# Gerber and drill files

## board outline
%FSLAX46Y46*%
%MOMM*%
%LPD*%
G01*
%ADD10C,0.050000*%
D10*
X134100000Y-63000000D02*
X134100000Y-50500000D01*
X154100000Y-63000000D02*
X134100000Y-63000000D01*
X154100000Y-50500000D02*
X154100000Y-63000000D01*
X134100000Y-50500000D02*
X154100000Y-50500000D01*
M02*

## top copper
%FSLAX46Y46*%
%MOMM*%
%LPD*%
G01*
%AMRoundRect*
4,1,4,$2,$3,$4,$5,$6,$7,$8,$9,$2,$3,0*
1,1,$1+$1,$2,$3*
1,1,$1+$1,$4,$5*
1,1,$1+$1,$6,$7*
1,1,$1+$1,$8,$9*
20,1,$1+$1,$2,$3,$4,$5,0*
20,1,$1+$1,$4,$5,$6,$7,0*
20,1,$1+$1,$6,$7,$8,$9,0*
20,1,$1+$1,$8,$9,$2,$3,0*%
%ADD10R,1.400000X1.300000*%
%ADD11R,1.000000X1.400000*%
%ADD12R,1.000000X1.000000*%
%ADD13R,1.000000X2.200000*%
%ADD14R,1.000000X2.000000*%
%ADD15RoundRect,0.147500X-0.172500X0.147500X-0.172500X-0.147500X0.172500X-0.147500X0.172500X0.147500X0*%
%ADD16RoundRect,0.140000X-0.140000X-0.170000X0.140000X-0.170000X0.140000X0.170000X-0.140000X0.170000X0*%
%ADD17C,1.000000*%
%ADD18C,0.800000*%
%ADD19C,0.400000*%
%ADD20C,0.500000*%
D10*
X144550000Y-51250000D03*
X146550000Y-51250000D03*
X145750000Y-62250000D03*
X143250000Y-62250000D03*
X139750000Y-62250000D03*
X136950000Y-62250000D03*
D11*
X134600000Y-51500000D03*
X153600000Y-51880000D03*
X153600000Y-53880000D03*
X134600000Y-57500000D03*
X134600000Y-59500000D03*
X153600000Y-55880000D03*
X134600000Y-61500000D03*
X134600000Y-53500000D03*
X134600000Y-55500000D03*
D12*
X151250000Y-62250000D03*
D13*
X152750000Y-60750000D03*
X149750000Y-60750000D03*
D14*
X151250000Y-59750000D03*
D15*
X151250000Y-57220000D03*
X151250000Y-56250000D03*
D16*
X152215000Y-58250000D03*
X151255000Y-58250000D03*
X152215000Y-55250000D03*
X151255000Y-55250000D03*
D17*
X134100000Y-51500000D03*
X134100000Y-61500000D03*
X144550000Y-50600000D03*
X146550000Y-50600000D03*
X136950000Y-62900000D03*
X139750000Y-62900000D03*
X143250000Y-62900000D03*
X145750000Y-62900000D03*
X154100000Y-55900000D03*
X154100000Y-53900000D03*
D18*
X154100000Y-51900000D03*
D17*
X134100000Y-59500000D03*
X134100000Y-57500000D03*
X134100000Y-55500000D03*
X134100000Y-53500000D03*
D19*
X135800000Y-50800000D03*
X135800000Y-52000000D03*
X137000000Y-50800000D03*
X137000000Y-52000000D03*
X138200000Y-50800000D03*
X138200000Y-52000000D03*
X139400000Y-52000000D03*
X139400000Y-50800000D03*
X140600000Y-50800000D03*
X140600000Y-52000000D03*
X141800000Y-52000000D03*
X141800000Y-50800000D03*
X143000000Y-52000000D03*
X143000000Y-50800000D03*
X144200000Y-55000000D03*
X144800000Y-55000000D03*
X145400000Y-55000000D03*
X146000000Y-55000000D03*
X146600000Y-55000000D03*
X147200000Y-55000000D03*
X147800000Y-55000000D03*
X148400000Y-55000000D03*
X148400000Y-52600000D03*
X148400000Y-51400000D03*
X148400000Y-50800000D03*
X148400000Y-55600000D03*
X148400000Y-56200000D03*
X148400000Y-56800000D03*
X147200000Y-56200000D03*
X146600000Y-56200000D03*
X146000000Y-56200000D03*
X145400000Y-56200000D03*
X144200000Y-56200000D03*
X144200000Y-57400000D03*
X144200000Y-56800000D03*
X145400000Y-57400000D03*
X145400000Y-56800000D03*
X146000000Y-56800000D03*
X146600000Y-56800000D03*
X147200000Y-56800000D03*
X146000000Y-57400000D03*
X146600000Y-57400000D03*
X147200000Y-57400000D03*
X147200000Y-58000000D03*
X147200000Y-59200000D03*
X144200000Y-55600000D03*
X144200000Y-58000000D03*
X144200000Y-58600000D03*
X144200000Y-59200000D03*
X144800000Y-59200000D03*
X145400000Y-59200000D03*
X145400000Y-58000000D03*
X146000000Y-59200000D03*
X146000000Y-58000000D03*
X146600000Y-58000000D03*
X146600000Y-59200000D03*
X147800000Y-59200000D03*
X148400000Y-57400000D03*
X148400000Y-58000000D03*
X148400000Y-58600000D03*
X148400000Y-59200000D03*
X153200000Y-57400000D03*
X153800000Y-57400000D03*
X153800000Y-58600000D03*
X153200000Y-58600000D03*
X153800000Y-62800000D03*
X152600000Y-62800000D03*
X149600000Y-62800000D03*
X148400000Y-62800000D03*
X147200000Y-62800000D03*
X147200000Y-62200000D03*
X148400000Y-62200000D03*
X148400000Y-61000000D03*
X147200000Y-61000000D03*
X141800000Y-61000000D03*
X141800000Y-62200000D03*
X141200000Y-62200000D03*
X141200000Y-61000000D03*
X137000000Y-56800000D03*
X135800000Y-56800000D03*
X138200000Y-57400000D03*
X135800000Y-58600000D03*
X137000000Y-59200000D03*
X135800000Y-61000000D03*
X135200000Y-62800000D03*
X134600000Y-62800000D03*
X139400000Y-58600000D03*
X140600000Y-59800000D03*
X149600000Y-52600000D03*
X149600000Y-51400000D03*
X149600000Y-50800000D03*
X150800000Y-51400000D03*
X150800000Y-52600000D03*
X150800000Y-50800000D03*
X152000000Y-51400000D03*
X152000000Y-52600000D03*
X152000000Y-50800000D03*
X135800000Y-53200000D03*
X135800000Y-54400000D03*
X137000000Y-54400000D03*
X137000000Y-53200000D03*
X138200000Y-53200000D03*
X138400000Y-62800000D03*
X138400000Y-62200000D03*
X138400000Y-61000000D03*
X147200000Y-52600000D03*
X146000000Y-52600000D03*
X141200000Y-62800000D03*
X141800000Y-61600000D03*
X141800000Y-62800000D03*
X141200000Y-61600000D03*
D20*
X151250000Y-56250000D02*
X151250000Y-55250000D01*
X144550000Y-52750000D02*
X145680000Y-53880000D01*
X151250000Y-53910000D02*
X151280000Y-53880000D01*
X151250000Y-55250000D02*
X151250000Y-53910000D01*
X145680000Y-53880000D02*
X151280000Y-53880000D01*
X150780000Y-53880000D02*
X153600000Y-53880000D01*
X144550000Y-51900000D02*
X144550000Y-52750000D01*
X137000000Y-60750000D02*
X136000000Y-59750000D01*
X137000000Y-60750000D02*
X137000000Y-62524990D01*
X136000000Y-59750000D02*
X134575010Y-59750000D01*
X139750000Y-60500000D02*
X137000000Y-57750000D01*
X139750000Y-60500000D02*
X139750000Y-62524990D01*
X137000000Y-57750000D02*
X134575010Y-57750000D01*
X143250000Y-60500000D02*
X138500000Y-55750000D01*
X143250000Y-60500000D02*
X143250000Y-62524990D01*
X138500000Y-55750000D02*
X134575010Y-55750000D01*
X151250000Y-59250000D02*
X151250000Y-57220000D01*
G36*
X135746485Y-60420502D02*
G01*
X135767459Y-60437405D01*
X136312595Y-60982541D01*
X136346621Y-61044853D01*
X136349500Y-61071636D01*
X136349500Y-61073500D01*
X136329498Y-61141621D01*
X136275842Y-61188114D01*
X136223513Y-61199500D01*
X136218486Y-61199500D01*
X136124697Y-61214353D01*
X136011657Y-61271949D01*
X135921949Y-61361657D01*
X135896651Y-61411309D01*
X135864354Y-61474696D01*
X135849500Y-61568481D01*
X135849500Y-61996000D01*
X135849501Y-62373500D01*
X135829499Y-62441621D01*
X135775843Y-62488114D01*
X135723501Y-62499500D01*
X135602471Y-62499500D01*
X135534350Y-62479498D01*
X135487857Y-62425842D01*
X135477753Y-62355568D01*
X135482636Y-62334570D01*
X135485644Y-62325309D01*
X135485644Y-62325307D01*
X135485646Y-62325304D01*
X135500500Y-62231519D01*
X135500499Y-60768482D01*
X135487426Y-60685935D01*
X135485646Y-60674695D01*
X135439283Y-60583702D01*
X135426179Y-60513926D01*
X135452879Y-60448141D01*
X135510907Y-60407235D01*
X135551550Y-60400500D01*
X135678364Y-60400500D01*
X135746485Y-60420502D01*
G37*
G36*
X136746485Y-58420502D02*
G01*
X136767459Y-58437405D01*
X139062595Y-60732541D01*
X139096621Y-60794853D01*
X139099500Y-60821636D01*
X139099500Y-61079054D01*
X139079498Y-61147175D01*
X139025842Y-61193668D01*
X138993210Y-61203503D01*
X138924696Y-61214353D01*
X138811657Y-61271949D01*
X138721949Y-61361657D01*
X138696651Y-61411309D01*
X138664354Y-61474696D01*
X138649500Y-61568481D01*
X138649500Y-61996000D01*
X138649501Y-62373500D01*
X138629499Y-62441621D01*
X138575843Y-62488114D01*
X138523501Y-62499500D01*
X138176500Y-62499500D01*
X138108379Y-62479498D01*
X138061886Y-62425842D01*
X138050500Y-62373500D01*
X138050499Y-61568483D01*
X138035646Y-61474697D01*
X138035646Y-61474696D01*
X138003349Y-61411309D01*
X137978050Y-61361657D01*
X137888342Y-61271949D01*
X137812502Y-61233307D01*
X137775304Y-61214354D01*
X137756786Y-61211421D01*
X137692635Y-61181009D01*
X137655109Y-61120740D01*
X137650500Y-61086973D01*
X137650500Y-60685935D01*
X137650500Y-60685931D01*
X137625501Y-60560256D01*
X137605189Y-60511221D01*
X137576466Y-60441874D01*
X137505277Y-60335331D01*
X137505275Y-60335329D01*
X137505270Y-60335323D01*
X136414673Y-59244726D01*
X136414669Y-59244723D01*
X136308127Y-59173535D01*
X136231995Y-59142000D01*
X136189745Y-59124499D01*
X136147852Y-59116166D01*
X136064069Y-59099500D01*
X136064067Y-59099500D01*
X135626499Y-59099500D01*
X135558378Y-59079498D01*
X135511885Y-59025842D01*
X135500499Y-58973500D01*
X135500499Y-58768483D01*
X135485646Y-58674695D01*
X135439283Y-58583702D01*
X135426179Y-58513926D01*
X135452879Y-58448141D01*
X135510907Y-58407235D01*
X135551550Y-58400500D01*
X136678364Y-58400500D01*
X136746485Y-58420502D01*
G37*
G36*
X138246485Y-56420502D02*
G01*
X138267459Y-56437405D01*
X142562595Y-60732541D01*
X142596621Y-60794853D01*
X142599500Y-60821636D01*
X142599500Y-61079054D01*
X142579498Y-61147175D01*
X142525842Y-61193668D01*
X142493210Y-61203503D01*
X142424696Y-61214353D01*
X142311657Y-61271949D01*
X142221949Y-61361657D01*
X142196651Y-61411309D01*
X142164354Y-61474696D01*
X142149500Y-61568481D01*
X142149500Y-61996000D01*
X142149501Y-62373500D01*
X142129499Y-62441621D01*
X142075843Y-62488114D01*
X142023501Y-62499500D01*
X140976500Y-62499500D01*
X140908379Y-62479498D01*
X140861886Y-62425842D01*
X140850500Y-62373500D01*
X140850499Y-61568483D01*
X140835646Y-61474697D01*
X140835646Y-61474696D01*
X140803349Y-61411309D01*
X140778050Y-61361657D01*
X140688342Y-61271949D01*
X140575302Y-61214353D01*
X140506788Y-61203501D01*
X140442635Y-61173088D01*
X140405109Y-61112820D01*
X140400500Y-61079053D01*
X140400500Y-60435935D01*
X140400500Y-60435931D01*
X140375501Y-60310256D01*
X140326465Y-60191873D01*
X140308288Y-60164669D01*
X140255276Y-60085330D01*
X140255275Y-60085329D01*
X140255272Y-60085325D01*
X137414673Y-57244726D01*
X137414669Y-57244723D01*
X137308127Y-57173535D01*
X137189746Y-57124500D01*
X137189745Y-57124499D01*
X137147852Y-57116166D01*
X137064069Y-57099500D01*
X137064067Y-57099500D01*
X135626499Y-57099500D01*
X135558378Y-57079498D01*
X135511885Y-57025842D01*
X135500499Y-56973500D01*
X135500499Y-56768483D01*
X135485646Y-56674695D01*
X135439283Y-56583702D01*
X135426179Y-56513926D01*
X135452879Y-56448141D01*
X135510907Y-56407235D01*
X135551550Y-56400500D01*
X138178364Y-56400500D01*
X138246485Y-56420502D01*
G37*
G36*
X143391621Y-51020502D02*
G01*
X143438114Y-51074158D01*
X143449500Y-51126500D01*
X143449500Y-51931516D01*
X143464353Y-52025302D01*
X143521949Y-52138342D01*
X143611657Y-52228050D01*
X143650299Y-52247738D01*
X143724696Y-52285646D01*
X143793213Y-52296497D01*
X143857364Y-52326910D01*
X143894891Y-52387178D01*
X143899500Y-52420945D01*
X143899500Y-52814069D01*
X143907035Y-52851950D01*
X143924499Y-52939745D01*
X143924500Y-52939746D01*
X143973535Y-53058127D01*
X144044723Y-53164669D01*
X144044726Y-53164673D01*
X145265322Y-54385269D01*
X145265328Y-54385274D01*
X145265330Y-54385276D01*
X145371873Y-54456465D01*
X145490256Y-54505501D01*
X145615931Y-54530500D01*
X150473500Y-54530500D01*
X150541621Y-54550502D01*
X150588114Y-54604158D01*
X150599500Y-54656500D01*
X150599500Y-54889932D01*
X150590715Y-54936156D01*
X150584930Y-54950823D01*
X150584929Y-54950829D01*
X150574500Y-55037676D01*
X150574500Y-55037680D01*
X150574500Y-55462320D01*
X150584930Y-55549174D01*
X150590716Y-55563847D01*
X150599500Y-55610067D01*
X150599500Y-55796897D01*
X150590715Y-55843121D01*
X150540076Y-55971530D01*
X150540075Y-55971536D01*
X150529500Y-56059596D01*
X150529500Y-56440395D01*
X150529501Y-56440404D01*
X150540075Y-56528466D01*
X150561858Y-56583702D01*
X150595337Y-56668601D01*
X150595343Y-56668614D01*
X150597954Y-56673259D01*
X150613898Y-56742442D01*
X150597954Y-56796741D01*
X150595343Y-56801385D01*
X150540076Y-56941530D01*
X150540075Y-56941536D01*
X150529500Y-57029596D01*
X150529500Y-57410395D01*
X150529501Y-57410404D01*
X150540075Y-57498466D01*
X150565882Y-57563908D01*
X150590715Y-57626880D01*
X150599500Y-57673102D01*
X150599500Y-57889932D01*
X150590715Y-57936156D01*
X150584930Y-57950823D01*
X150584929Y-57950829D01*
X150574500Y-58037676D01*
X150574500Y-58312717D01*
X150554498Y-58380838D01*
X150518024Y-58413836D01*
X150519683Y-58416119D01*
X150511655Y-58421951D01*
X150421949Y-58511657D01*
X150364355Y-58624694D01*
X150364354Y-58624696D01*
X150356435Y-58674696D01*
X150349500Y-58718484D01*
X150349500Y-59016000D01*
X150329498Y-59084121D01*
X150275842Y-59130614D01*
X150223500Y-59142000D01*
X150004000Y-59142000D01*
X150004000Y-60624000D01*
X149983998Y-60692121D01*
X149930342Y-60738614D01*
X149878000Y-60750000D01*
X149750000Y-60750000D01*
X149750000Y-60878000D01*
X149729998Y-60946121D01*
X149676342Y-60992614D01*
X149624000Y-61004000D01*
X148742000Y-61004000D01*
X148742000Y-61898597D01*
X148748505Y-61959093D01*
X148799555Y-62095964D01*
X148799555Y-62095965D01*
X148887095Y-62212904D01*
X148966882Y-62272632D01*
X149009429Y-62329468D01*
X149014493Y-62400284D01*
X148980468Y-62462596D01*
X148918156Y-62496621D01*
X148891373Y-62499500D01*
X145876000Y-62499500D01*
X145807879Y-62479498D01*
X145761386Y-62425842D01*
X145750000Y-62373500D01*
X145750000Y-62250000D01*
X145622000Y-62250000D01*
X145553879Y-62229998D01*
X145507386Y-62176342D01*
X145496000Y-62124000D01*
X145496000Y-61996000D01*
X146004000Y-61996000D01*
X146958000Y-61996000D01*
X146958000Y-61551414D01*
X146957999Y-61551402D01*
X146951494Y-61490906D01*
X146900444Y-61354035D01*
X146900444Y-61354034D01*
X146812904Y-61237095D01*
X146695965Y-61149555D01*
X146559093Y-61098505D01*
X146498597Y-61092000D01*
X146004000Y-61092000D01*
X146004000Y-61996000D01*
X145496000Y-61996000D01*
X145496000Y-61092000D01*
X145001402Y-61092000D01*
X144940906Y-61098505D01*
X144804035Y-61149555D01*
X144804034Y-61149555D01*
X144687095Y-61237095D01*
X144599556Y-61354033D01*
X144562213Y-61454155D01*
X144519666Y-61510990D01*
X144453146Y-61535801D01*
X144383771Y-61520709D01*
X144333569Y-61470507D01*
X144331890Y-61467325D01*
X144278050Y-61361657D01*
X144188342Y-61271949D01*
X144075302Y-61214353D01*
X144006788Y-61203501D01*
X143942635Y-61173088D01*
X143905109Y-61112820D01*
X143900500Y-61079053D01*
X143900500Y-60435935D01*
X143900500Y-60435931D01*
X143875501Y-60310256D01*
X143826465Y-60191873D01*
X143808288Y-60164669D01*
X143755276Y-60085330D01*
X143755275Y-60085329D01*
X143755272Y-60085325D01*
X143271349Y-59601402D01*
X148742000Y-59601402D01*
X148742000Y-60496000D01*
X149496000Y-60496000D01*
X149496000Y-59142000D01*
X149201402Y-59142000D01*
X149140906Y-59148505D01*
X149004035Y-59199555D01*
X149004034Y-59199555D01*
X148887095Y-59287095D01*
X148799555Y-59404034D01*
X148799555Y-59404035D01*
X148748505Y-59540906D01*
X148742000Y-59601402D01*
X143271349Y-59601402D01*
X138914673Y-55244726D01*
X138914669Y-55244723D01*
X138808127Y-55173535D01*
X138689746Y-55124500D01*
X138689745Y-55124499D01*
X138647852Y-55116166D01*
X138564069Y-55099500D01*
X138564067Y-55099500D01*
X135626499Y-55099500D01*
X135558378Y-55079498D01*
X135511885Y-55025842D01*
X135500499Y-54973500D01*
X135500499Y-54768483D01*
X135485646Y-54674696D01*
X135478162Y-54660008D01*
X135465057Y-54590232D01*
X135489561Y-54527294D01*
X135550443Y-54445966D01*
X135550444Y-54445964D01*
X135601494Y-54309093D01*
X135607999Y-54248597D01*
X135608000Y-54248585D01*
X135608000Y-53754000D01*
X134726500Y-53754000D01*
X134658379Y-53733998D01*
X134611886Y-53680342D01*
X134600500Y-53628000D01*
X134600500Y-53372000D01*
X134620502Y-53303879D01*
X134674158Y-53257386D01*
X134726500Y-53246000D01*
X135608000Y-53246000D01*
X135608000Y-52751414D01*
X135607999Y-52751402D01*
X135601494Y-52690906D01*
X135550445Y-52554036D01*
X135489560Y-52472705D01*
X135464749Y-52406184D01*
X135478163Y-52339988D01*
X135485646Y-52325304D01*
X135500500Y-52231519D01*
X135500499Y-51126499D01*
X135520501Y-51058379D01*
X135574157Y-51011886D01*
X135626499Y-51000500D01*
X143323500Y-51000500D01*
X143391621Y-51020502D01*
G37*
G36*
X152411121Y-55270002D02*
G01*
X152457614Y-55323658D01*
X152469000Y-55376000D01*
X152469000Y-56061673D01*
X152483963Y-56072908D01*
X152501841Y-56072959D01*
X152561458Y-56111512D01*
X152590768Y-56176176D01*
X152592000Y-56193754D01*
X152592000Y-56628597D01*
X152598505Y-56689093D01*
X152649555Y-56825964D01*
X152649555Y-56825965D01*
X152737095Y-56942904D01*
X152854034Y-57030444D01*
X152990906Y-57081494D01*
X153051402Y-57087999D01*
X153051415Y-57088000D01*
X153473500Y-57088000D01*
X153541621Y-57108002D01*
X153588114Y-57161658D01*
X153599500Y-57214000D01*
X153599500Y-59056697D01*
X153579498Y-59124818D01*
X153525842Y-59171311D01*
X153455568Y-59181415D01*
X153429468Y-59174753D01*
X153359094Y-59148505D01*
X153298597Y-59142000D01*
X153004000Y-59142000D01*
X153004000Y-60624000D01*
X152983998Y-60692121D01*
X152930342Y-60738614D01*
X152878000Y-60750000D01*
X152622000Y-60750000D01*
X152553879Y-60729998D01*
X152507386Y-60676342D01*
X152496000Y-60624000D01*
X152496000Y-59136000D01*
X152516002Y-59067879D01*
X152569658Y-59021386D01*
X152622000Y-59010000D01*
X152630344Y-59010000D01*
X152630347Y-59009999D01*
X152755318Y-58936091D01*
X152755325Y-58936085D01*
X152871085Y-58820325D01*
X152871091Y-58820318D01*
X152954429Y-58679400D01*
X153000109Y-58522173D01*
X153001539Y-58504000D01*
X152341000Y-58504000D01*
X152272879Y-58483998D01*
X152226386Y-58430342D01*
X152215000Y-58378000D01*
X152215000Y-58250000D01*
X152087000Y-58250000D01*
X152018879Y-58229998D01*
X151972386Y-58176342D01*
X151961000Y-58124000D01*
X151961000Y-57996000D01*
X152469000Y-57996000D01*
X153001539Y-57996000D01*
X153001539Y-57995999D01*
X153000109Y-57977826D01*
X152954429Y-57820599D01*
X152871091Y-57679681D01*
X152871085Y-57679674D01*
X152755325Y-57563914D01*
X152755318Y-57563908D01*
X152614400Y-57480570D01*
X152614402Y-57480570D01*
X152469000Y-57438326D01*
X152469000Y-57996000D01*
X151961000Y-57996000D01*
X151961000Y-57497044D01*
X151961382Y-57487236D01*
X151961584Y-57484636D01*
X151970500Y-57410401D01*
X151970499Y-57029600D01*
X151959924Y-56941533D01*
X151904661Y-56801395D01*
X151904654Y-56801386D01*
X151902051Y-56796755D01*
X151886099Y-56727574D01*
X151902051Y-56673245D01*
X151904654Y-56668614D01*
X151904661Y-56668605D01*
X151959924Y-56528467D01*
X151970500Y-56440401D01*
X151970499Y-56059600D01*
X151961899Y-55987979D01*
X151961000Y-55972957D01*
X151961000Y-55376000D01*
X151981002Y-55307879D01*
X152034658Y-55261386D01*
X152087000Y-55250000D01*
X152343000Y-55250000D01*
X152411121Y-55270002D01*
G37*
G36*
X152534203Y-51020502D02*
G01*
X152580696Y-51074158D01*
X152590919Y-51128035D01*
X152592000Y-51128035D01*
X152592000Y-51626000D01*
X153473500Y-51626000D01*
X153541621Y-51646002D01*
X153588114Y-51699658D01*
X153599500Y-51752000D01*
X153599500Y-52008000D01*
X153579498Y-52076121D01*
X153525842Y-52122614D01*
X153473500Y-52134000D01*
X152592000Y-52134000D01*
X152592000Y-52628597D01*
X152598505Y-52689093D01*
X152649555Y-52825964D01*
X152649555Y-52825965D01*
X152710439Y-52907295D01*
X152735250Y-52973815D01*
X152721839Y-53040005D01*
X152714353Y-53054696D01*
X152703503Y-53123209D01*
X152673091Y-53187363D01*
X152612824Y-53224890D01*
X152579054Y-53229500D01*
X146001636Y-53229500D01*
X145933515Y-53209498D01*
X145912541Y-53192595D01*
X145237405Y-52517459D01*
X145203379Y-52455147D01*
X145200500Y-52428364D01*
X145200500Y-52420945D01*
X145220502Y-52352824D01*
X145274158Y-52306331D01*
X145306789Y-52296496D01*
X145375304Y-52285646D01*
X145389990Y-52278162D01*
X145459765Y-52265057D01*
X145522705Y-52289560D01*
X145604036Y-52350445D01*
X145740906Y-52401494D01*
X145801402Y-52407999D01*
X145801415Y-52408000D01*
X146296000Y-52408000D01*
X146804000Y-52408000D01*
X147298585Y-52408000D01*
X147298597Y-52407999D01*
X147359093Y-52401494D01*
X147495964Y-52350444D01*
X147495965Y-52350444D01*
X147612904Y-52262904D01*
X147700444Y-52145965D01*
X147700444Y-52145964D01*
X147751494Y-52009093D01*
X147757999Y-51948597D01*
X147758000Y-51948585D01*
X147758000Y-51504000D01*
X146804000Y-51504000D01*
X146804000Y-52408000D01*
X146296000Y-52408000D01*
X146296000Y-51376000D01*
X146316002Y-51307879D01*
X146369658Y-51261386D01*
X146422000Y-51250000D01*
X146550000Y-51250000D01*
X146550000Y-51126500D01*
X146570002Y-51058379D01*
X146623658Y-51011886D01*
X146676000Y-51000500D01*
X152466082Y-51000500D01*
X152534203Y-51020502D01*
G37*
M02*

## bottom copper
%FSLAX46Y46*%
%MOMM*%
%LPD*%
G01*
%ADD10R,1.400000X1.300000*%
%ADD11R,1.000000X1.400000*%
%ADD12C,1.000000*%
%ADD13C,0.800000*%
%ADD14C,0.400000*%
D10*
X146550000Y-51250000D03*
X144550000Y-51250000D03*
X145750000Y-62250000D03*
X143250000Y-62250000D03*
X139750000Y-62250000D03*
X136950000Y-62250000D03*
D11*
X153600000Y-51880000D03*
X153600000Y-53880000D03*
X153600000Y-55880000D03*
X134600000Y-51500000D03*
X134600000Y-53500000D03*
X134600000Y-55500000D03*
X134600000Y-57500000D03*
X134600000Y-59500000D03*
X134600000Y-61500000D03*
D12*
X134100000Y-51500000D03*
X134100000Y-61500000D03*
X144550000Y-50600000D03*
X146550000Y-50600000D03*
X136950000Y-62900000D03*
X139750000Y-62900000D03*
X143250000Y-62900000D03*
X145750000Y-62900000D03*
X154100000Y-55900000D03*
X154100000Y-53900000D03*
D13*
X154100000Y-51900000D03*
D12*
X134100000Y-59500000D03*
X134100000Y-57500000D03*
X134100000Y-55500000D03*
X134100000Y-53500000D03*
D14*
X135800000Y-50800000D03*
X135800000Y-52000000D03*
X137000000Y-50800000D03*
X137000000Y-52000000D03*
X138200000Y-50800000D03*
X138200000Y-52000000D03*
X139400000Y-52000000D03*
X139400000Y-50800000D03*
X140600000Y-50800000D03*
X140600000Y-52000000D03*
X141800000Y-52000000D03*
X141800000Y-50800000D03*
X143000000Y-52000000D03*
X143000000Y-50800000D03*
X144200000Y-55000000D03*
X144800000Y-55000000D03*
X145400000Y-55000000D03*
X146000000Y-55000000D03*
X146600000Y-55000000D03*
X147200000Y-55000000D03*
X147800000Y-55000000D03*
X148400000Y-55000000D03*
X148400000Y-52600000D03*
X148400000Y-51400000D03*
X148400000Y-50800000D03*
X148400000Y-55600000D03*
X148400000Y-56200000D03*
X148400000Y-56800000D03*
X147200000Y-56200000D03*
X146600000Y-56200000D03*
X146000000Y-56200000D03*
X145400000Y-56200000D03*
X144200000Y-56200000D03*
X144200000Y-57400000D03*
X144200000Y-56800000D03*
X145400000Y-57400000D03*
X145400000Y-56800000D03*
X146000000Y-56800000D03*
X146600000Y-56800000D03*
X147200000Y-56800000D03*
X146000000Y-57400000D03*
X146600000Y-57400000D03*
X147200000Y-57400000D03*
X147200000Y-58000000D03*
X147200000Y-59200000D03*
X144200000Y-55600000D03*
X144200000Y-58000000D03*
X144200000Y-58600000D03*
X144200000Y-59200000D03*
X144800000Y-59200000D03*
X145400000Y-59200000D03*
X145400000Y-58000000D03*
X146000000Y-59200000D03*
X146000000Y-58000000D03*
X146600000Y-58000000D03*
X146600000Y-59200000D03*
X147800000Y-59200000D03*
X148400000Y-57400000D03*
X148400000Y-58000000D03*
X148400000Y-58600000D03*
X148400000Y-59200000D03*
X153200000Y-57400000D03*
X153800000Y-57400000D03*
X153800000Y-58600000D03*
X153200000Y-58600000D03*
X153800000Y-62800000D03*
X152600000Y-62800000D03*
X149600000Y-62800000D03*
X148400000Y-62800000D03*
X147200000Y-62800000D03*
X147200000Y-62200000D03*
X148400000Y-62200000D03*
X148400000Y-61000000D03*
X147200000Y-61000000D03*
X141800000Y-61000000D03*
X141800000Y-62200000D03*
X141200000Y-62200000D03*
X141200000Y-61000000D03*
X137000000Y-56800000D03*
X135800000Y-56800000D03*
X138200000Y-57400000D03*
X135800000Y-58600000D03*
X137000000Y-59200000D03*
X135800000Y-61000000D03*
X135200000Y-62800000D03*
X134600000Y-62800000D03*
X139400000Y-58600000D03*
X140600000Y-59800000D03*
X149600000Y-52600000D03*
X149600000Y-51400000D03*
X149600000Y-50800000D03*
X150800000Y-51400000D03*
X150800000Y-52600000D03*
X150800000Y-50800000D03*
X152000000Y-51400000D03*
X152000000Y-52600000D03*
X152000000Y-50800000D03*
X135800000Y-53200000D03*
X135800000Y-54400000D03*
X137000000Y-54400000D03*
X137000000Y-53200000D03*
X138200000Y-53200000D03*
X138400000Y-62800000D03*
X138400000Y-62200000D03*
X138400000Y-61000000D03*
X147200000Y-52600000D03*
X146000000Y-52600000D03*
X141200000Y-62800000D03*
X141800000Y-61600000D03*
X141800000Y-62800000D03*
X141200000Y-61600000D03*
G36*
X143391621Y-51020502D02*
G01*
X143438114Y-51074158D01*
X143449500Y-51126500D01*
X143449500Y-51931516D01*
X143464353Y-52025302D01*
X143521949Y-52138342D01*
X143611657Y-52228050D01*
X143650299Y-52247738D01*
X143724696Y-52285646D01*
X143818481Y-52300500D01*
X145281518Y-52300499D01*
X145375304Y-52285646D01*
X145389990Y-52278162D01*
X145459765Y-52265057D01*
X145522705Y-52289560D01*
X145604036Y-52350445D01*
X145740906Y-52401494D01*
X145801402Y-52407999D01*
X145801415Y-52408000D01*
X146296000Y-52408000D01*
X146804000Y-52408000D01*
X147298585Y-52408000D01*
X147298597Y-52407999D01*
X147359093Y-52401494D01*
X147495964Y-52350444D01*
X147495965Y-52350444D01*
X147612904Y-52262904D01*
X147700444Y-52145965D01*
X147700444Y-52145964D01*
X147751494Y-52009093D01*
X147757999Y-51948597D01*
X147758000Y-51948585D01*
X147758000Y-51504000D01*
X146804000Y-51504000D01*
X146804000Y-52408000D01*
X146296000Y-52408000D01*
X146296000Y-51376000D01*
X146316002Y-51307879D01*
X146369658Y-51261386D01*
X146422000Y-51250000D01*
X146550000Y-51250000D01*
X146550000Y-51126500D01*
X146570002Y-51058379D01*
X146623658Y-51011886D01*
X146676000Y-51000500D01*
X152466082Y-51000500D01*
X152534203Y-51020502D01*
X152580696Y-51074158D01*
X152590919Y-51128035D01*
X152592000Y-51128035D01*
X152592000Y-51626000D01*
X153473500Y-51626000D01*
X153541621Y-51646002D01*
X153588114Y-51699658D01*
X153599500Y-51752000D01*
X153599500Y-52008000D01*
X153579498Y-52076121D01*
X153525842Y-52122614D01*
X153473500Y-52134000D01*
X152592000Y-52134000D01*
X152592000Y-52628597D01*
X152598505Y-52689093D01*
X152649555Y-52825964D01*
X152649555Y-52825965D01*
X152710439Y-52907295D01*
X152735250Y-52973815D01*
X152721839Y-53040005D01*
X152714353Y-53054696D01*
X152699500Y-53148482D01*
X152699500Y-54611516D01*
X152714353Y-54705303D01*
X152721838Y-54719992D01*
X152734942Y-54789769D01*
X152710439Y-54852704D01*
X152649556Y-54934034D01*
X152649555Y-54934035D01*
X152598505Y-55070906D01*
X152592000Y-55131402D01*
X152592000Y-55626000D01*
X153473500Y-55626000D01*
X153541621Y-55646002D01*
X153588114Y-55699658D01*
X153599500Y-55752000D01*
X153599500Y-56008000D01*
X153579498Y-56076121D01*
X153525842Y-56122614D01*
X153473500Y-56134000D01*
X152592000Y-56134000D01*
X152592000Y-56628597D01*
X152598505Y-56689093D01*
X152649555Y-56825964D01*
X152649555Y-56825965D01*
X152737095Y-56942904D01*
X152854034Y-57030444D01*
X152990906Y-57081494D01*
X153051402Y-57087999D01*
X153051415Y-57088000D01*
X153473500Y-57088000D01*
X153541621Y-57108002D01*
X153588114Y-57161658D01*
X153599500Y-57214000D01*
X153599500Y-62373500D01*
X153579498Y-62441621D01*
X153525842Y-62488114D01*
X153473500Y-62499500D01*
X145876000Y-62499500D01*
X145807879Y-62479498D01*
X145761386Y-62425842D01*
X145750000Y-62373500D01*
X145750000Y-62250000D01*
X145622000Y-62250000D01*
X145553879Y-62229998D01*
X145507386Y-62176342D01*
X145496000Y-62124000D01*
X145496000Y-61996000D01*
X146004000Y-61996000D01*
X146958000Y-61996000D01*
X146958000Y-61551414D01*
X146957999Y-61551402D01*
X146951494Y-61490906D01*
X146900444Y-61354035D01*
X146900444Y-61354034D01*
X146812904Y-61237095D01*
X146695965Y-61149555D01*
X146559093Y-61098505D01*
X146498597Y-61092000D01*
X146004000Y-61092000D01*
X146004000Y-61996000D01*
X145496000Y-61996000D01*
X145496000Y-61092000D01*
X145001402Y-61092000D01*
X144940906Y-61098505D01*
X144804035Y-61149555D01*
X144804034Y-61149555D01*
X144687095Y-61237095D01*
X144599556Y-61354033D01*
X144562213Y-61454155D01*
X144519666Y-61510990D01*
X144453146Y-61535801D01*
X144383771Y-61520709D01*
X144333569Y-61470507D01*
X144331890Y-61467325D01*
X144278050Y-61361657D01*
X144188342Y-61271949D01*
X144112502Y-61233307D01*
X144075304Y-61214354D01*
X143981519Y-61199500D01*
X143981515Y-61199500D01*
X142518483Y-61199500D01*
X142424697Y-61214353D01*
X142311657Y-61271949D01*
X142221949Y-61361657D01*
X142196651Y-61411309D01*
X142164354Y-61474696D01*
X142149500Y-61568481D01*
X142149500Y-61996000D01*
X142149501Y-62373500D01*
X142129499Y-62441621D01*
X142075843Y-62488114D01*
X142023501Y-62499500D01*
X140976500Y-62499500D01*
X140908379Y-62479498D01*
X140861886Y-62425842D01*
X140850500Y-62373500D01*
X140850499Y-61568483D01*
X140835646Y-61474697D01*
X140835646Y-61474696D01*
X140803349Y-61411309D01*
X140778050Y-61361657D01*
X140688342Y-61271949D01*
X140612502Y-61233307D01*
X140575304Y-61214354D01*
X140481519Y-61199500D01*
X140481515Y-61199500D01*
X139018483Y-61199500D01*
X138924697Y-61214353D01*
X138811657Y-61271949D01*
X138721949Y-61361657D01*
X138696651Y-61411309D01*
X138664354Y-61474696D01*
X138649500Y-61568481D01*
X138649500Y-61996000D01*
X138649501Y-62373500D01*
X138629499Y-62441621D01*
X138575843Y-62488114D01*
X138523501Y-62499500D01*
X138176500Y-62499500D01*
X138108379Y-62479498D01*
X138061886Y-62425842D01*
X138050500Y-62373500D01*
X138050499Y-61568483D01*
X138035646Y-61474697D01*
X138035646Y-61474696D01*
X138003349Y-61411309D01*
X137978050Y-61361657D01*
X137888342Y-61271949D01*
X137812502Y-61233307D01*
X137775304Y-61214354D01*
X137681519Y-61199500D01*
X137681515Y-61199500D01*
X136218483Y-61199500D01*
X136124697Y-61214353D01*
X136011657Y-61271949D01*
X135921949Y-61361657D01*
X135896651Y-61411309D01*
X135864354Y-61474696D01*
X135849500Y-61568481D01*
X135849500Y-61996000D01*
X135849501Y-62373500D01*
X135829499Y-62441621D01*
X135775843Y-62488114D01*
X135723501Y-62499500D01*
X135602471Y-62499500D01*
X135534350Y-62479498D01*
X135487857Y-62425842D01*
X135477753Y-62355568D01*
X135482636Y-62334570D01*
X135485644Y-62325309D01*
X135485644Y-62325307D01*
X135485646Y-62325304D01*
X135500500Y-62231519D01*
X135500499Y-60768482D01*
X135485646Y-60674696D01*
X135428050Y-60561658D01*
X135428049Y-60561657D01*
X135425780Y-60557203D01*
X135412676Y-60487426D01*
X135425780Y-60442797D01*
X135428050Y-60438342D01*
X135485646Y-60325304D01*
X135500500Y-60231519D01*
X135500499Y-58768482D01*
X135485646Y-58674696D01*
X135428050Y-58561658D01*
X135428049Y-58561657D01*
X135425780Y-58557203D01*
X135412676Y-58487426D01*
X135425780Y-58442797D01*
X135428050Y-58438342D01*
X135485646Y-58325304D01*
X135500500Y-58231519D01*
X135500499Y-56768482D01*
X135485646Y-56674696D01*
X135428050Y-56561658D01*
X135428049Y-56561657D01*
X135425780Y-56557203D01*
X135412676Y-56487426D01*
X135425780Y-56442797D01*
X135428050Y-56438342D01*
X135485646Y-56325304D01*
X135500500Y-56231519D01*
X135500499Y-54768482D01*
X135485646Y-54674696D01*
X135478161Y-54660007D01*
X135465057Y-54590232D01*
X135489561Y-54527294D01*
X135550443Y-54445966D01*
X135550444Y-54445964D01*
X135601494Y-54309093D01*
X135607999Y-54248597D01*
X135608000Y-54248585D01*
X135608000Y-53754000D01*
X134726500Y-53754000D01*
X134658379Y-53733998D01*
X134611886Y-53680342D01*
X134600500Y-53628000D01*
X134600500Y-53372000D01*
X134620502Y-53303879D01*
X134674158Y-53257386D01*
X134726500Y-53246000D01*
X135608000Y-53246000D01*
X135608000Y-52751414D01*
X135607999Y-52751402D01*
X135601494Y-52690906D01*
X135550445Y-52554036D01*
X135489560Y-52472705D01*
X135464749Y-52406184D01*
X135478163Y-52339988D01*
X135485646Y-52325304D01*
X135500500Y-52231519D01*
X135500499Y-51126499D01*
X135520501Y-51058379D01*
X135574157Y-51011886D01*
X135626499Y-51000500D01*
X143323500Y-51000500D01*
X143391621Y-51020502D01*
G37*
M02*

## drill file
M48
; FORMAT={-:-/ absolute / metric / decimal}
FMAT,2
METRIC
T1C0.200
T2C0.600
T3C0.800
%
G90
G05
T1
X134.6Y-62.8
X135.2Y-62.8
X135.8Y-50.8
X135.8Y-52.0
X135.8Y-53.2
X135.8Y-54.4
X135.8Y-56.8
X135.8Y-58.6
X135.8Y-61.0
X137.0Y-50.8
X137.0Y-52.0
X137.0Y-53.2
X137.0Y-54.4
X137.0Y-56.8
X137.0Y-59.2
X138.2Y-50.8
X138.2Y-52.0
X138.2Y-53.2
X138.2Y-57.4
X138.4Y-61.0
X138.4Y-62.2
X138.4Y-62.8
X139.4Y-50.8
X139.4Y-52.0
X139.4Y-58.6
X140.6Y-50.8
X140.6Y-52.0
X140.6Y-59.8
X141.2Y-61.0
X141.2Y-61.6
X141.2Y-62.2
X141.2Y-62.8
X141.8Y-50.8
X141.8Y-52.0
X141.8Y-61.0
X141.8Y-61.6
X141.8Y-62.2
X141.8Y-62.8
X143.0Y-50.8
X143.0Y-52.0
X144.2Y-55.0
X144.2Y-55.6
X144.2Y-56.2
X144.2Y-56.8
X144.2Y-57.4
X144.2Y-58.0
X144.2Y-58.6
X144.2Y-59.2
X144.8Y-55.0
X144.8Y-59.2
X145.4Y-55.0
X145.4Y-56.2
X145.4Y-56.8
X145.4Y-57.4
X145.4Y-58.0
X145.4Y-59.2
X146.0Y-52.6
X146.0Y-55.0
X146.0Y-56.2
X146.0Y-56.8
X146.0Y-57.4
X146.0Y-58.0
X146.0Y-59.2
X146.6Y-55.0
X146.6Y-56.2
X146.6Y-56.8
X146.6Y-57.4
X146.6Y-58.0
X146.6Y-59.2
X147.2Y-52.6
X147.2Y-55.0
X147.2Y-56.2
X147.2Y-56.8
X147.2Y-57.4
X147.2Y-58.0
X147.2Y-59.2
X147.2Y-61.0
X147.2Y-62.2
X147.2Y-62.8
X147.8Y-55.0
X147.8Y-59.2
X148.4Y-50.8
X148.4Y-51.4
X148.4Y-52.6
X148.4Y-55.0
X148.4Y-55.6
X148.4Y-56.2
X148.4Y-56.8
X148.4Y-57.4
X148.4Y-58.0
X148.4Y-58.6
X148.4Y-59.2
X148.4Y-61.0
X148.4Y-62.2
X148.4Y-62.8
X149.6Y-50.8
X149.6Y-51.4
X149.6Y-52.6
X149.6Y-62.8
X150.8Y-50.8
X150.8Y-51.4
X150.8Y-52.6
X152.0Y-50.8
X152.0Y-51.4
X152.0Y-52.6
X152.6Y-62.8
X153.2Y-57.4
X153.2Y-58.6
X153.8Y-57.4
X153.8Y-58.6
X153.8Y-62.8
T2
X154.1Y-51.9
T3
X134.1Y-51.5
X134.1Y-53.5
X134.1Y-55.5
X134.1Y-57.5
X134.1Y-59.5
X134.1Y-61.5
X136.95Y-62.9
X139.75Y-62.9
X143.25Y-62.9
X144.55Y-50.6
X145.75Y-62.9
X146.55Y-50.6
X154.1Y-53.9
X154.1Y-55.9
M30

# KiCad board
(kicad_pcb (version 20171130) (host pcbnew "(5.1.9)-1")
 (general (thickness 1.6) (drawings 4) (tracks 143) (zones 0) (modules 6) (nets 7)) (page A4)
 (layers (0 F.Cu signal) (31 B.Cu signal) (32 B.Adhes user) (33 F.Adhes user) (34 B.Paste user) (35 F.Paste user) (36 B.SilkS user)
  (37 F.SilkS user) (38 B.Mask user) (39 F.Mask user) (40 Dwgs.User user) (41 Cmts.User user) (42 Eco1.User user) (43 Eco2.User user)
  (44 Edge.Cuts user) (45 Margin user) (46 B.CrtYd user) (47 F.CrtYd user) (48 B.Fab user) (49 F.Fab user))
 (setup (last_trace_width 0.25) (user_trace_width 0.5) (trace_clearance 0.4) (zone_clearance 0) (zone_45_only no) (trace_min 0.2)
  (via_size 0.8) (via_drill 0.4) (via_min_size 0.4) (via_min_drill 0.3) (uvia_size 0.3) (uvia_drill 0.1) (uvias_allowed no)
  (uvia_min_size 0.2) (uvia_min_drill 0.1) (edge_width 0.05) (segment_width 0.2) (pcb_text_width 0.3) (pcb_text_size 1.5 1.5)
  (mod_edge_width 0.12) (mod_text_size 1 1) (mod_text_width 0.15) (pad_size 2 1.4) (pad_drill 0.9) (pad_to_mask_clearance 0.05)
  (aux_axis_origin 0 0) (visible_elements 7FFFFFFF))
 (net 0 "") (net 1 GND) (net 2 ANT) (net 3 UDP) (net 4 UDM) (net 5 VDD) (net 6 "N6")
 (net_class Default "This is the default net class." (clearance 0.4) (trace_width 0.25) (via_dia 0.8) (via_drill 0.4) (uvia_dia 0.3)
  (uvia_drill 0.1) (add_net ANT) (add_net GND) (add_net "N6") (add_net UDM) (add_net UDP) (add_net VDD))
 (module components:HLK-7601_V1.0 (layer F.Cu) (at 135.75 62.9 90)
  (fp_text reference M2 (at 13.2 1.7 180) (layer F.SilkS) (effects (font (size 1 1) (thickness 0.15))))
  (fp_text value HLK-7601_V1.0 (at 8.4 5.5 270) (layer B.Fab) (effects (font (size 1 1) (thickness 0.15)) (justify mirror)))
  (pad 5 smd rect (at 12.3 10.8 90) (size 1.3 1.4) (drill (offset -0.65 0)) (layers B.Cu B.Paste B.Mask) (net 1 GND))
  (pad 6 smd rect (at 12.3 8.8 90) (size 1.3 1.4) (drill (offset -0.65 0)) (layers B.Cu B.Paste B.Mask) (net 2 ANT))
  (pad 4 smd rect (at 0 10 90) (size 1.3 1.4) (drill (offset 0.65 0)) (layers B.Cu B.Paste B.Mask) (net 1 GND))
  (pad 3 smd rect (at 0 7.5 90) (size 1.3 1.4) (drill (offset 0.65 0)) (layers B.Cu B.Paste B.Mask) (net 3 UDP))
  (pad 2 smd rect (at 0 4 90) (size 1.3 1.4) (drill (offset 0.65 0)) (layers B.Cu B.Paste B.Mask) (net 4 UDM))
  (pad 1 smd rect (at 0 1.2 90) (size 1.3 1.4) (drill (offset 0.65 0)) (layers B.Cu B.Paste B.Mask) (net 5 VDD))
  (pad 6 smd rect (at 12.3 8.8 90) (size 1.3 1.4) (drill (offset -0.65 0)) (layers F.Cu F.Paste F.Mask) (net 2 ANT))
  (pad 5 smd rect (at 12.3 10.8 90) (size 1.3 1.4) (drill (offset -0.65 0)) (layers F.Cu F.Paste F.Mask) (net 1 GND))
  (pad 4 smd rect (at 0 10 90) (size 1.3 1.4) (drill (offset 0.65 0)) (layers F.Cu F.Paste F.Mask) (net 1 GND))
  (pad 3 smd rect (at 0 7.5 90) (size 1.3 1.4) (drill (offset 0.65 0)) (layers F.Cu F.Paste F.Mask) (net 3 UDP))
  (pad 2 smd rect (at 0 4 90) (size 1.3 1.4) (drill (offset 0.65 0)) (layers F.Cu F.Paste F.Mask) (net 4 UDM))
  (pad 1 smd rect (at 0 1.2 90) (size 1.3 1.4) (drill (offset 0.65 0)) (layers F.Cu F.Paste F.Mask) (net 5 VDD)))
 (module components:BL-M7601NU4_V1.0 (layer F.Cu) (at 134.1 50.5)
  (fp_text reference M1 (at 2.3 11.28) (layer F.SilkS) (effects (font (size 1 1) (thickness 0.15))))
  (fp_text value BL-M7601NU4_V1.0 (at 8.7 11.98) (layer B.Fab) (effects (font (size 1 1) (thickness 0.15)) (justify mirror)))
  (pad 6 smd rect (at 0 1) (size 1 1.4) (drill (offset 0.5 0)) (layers F.Cu F.Paste F.Mask))
  (pad 9 smd rect (at 20 1.38) (size 1 1.4) (drill (offset -0.5 0)) (layers F.Cu F.Paste F.Mask) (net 1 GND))
  (pad 8 smd rect (at 20 3.38) (size 1 1.4) (drill (offset -0.5 0)) (layers F.Cu F.Paste F.Mask) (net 2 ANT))
  (pad 3 smd rect (at 0 7) (size 1 1.4) (drill (offset 0.5 0)) (layers F.Cu F.Paste F.Mask) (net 4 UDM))
  (pad 2 smd rect (at 0 9) (size 1 1.4) (drill (offset 0.5 0)) (layers F.Cu F.Paste F.Mask) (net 5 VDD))
  (pad 7 smd rect (at 20 5.38) (size 1 1.4) (drill (offset -0.5 0)) (layers F.Cu F.Paste F.Mask) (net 1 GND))
  (pad 1 smd rect (at 0 11) (size 1 1.4) (drill (offset 0.5 0)) (layers F.Cu F.Paste F.Mask))
  (pad 5 smd rect (at 0 3) (size 1 1.4) (drill (offset 0.5 0)) (layers F.Cu F.Paste F.Mask) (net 1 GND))
  (pad 4 smd rect (at 0 5) (size 1 1.4) (drill (offset 0.5 0)) (layers F.Cu F.Paste F.Mask) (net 3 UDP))
  (pad 9 smd rect (at 20 1.38) (size 1 1.4) (drill (offset -0.5 0)) (layers B.Cu B.Paste B.Mask) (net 1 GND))
  (pad 8 smd rect (at 20 3.38) (size 1 1.4) (drill (offset -0.5 0)) (layers B.Cu B.Paste B.Mask) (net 2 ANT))
  (pad 7 smd rect (at 20 5.38) (size 1 1.4) (drill (offset -0.5 0)) (layers B.Cu B.Paste B.Mask) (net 1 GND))
  (pad 6 smd rect (at 0 1) (size 1 1.4) (drill (offset 0.5 0)) (layers B.Cu B.Paste B.Mask))
  (pad 5 smd rect (at 0 3) (size 1 1.4) (drill (offset 0.5 0)) (layers B.Cu B.Paste B.Mask) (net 1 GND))
  (pad 4 smd rect (at 0 5) (size 1 1.4) (drill (offset 0.5 0)) (layers B.Cu B.Paste B.Mask) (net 3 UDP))
  (pad 3 smd rect (at 0 7) (size 1 1.4) (drill (offset 0.5 0)) (layers B.Cu B.Paste B.Mask) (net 4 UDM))
  (pad 2 smd rect (at 0 9) (size 1 1.4) (drill (offset 0.5 0)) (layers B.Cu B.Paste B.Mask) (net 5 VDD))
  (pad 1 smd rect (at 0 11) (size 1 1.4) (drill (offset 0.5 0)) (layers B.Cu B.Paste B.Mask)))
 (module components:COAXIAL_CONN (layer F.Cu) (at 151.25 60.75 180)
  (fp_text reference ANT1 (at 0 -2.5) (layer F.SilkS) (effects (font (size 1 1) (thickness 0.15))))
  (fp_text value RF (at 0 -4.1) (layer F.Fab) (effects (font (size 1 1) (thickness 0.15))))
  (pad 4 smd rect (at 0 -1.5 180) (size 1 1) (layers F.Cu F.Paste F.Mask) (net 1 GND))
  (pad 3 smd rect (at -1.5 0 180) (size 1 2.2) (layers F.Cu F.Paste F.Mask) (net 1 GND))
  (pad 2 smd rect (at 1.5 0 180) (size 1 2.2) (layers F.Cu F.Paste F.Mask) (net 1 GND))
  (pad 1 smd rect (at 0 1.5 180) (size 1 2) (drill (offset 0 -0.5)) (layers F.Cu F.Paste F.Mask) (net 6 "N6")))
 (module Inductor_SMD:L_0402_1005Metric (layer F.Cu) (at 151.25 56.735 270)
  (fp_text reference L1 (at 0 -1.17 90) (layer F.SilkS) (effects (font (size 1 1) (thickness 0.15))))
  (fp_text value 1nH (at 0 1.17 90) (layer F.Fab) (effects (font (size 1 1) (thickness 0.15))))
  (pad 2 smd roundrect (at 0.485 0 270) (size 0.59 0.64) (layers F.Cu F.Paste F.Mask) (roundrect_rratio 0.25) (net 6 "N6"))
  (pad 1 smd roundrect (at -0.485 0 270) (size 0.59 0.64) (layers F.Cu F.Paste F.Mask) (roundrect_rratio 0.25) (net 2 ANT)))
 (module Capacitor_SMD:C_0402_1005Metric (layer F.Cu) (at 151.735 58.25)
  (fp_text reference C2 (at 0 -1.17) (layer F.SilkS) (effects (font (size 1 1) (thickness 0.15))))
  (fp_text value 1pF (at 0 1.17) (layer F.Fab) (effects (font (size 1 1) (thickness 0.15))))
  (pad 2 smd roundrect (at 0.48 0) (size 0.56 0.62) (layers F.Cu F.Paste F.Mask) (roundrect_rratio 0.25) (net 1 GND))
  (pad 1 smd roundrect (at -0.48 0) (size 0.56 0.62) (layers F.Cu F.Paste F.Mask) (roundrect_rratio 0.25) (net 6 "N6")))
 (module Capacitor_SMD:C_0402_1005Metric (layer F.Cu) (at 151.735 55.25)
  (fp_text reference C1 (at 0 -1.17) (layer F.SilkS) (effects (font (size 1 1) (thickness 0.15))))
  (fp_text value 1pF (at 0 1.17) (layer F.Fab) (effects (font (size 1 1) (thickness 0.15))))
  (pad 2 smd roundrect (at 0.48 0) (size 0.56 0.62) (layers F.Cu F.Paste F.Mask) (roundrect_rratio 0.25) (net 1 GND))
  (pad 1 smd roundrect (at -0.48 0) (size 0.56 0.62) (layers F.Cu F.Paste F.Mask) (roundrect_rratio 0.25) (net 2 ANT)))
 (gr_line (start 134.1 63) (end 134.1 50.5) (layer Edge.Cuts) (width 0.05))
 (gr_line (start 154.1 63) (end 134.1 63) (layer Edge.Cuts) (width 0.05))
 (gr_line (start 154.1 50.5) (end 154.1 63) (layer Edge.Cuts) (width 0.05))
 (gr_line (start 134.1 50.5) (end 154.1 50.5) (layer Edge.Cuts) (width 0.05))
 (via (at 134.1 51.5) (size 1) (drill 0.8) (layers F.Cu B.Cu) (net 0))
 (via (at 134.1 61.5) (size 1) (drill 0.8) (layers F.Cu B.Cu) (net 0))
 (via (at 144.55 50.6) (size 1) (drill 0.8) (layers F.Cu B.Cu) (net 2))
 (via (at 146.55 50.6) (size 1) (drill 0.8) (layers F.Cu B.Cu) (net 1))
 (via (at 136.95 62.9) (size 1) (drill 0.8) (layers F.Cu B.Cu) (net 5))
 (via (at 139.75 62.9) (size 1) (drill 0.8) (layers F.Cu B.Cu) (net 4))
 (via (at 143.25 62.9) (size 1) (drill 0.8) (layers F.Cu B.Cu) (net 3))
 (via (at 145.75 62.9) (size 1) (drill 0.8) (layers F.Cu B.Cu) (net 1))
 (via (at 154.1 55.9) (size 1) (drill 0.8) (layers F.Cu B.Cu) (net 1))
 (via (at 154.1 53.9) (size 1) (drill 0.8) (layers F.Cu B.Cu) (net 2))
 (via (at 154.1 51.9) (size 0.8) (drill 0.6) (layers F.Cu B.Cu) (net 1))
 (via (at 134.1 59.5) (size 1) (drill 0.8) (layers F.Cu B.Cu) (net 5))
 (via (at 134.1 57.5) (size 1) (drill 0.8) (layers F.Cu B.Cu) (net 4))
 (via (at 134.1 55.5) (size 1) (drill 0.8) (layers F.Cu B.Cu) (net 3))
 (via (at 134.1 53.5) (size 1) (drill 0.8) (layers F.Cu B.Cu) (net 1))
 (segment (start 151.25 56.25) (end 151.25 55.25) (width 0.5) (layer F.Cu) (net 2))
 (segment (start 144.55 52.75) (end 145.68 53.88) (width 0.5) (layer F.Cu) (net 2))
 (segment (start 151.25 53.91) (end 151.28 53.88) (width 0.5) (layer F.Cu) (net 2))
 (segment (start 151.25 55.25) (end 151.25 53.91) (width 0.5) (layer F.Cu) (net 2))
 (segment (start 145.68 53.88) (end 151.28 53.88) (width 0.5) (layer F.Cu) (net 2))
 (segment (start 150.78 53.88) (end 153.6 53.88) (width 0.5) (layer F.Cu) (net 2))
 (segment (start 144.55 51.9) (end 144.55 52.75) (width 0.5) (layer F.Cu) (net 2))
 (via (at 135.8 50.8) (size 0.4) (drill 0.2) (layers F.Cu B.Cu) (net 1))
 (via (at 135.8 52) (size 0.4) (drill 0.2) (layers F.Cu B.Cu) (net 1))
 (via (at 137 50.8) (size 0.4) (drill 0.2) (layers F.Cu B.Cu) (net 1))
 (via (at 137 52) (size 0.4) (drill 0.2) (layers F.Cu B.Cu) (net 1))
 (via (at 138.2 50.8) (size 0.4) (drill 0.2) (layers F.Cu B.Cu) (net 1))
 (via (at 138.2 52) (size 0.4) (drill 0.2) (layers F.Cu B.Cu) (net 1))
 (via (at 139.4 52) (size 0.4) (drill 0.2) (layers F.Cu B.Cu) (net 1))
 (via (at 139.4 50.8) (size 0.4) (drill 0.2) (layers F.Cu B.Cu) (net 1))
 (via (at 140.6 50.8) (size 0.4) (drill 0.2) (layers F.Cu B.Cu) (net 1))
 (via (at 140.6 52) (size 0.4) (drill 0.2) (layers F.Cu B.Cu) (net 1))
 (via (at 141.8 52) (size 0.4) (drill 0.2) (layers F.Cu B.Cu) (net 1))
 (via (at 141.8 50.8) (size 0.4) (drill 0.2) (layers F.Cu B.Cu) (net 1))
 (via (at 143 52) (size 0.4) (drill 0.2) (layers F.Cu B.Cu) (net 1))
 (via (at 143 50.8) (size 0.4) (drill 0.2) (layers F.Cu B.Cu) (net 1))
 (via (at 144.2 55) (size 0.4) (drill 0.2) (layers F.Cu B.Cu) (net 1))
 (via (at 144.8 55) (size 0.4) (drill 0.2) (layers F.Cu B.Cu) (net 1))
 (via (at 145.4 55) (size 0.4) (drill 0.2) (layers F.Cu B.Cu) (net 1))
 (via (at 146 55) (size 0.4) (drill 0.2) (layers F.Cu B.Cu) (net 1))
 (via (at 146.6 55) (size 0.4) (drill 0.2) (layers F.Cu B.Cu) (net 1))
 (via (at 147.2 55) (size 0.4) (drill 0.2) (layers F.Cu B.Cu) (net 1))
 (via (at 147.8 55) (size 0.4) (drill 0.2) (layers F.Cu B.Cu) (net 1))
 (via (at 148.4 55) (size 0.4) (drill 0.2) (layers F.Cu B.Cu) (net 1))
 (via (at 148.4 52.6) (size 0.4) (drill 0.2) (layers F.Cu B.Cu) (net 1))
 (via (at 148.4 51.4) (size 0.4) (drill 0.2) (layers F.Cu B.Cu) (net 1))
 (via (at 148.4 50.8) (size 0.4) (drill 0.2) (layers F.Cu B.Cu) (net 1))
 (via (at 148.4 55.6) (size 0.4) (drill 0.2) (layers F.Cu B.Cu) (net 1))
 (via (at 148.4 56.2) (size 0.4) (drill 0.2) (layers F.Cu B.Cu) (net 1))
 (via (at 148.4 56.8) (size 0.4) (drill 0.2) (layers F.Cu B.Cu) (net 1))
 (via (at 147.2 56.2) (size 0.4) (drill 0.2) (layers F.Cu B.Cu) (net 1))
 (via (at 146.6 56.2) (size 0.4) (drill 0.2) (layers F.Cu B.Cu) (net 1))
 (via (at 146 56.2) (size 0.4) (drill 0.2) (layers F.Cu B.Cu) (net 1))
 (via (at 145.4 56.2) (size 0.4) (drill 0.2) (layers F.Cu B.Cu) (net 1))
 (via (at 144.2 56.2) (size 0.4) (drill 0.2) (layers F.Cu B.Cu) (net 1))
 (via (at 144.2 57.4) (size 0.4) (drill 0.2) (layers F.Cu B.Cu) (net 1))
 (via (at 144.2 56.8) (size 0.4) (drill 0.2) (layers F.Cu B.Cu) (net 1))
 (via (at 145.4 57.4) (size 0.4) (drill 0.2) (layers F.Cu B.Cu) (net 1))
 (via (at 145.4 56.8) (size 0.4) (drill 0.2) (layers F.Cu B.Cu) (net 1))
 (via (at 146 56.8) (size 0.4) (drill 0.2) (layers F.Cu B.Cu) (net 1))
 (via (at 146.6 56.8) (size 0.4) (drill 0.2) (layers F.Cu B.Cu) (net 1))
 (via (at 147.2 56.8) (size 0.4) (drill 0.2) (layers F.Cu B.Cu) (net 1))
 (via (at 146 57.4) (size 0.4) (drill 0.2) (layers F.Cu B.Cu) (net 1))
 (via (at 146.6 57.4) (size 0.4) (drill 0.2) (layers F.Cu B.Cu) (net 1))
 (via (at 147.2 57.4) (size 0.4) (drill 0.2) (layers F.Cu B.Cu) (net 1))
 (via (at 147.2 58) (size 0.4) (drill 0.2) (layers F.Cu B.Cu) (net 1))
 (via (at 147.2 59.2) (size 0.4) (drill 0.2) (layers F.Cu B.Cu) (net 1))
 (via (at 144.2 55.6) (size 0.4) (drill 0.2) (layers F.Cu B.Cu) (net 1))
 (via (at 144.2 58) (size 0.4) (drill 0.2) (layers F.Cu B.Cu) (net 1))
 (via (at 144.2 58.6) (size 0.4) (drill 0.2) (layers F.Cu B.Cu) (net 1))
 (via (at 144.2 59.2) (size 0.4) (drill 0.2) (layers F.Cu B.Cu) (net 1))
 (via (at 144.8 59.2) (size 0.4) (drill 0.2) (layers F.Cu B.Cu) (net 1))
 (via (at 145.4 59.2) (size 0.4) (drill 0.2) (layers F.Cu B.Cu) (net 1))
 (via (at 145.4 58) (size 0.4) (drill 0.2) (layers F.Cu B.Cu) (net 1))
 (via (at 146 59.2) (size 0.4) (drill 0.2) (layers F.Cu B.Cu) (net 1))
 (via (at 146 58) (size 0.4) (drill 0.2) (layers F.Cu B.Cu) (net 1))
 (via (at 146.6 58) (size 0.4) (drill 0.2) (layers F.Cu B.Cu) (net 1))
 (via (at 146.6 59.2) (size 0.4) (drill 0.2) (layers F.Cu B.Cu) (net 1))
 (via (at 147.8 59.2) (size 0.4) (drill 0.2) (layers F.Cu B.Cu) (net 1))
 (via (at 148.4 57.4) (size 0.4) (drill 0.2) (layers F.Cu B.Cu) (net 1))
 (via (at 148.4 58) (size 0.4) (drill 0.2) (layers F.Cu B.Cu) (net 1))
 (via (at 148.4 58.6) (size 0.4) (drill 0.2) (layers F.Cu B.Cu) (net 1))
 (via (at 148.4 59.2) (size 0.4) (drill 0.2) (layers F.Cu B.Cu) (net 1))
 (via (at 153.2 57.4) (size 0.4) (drill 0.2) (layers F.Cu B.Cu) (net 1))
 (via (at 153.8 57.4) (size 0.4) (drill 0.2) (layers F.Cu B.Cu) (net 1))
 (via (at 153.8 58.6) (size 0.4) (drill 0.2) (layers F.Cu B.Cu) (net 1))
 (via (at 153.2 58.6) (size 0.4) (drill 0.2) (layers F.Cu B.Cu) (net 1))
 (via (at 153.8 62.8) (size 0.4) (drill 0.2) (layers F.Cu B.Cu) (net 1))
 (via (at 152.6 62.8) (size 0.4) (drill 0.2) (layers F.Cu B.Cu) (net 1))
 (via (at 149.6 62.8) (size 0.4) (drill 0.2) (layers F.Cu B.Cu) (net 1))
 (via (at 148.4 62.8) (size 0.4) (drill 0.2) (layers F.Cu B.Cu) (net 1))
 (via (at 147.2 62.8) (size 0.4) (drill 0.2) (layers F.Cu B.Cu) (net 1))
 (via (at 147.2 62.2) (size 0.4) (drill 0.2) (layers F.Cu B.Cu) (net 1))
 (via (at 148.4 62.2) (size 0.4) (drill 0.2) (layers F.Cu B.Cu) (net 1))
 (via (at 148.4 61) (size 0.4) (drill 0.2) (layers F.Cu B.Cu) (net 1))
 (via (at 147.2 61) (size 0.4) (drill 0.2) (layers F.Cu B.Cu) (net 1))
 (via (at 141.8 61) (size 0.4) (drill 0.2) (layers F.Cu B.Cu) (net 1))
 (via (at 141.8 62.2) (size 0.4) (drill 0.2) (layers F.Cu B.Cu) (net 1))
 (via (at 141.2 62.2) (size 0.4) (drill 0.2) (layers F.Cu B.Cu) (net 1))
 (via (at 141.2 61) (size 0.4) (drill 0.2) (layers F.Cu B.Cu) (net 1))
 (via (at 137 56.8) (size 0.4) (drill 0.2) (layers F.Cu B.Cu) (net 1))
 (via (at 135.8 56.8) (size 0.4) (drill 0.2) (layers F.Cu B.Cu) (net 1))
 (via (at 138.2 57.4) (size 0.4) (drill 0.2) (layers F.Cu B.Cu) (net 1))
 (via (at 135.8 58.6) (size 0.4) (drill 0.2) (layers F.Cu B.Cu) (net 1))
 (via (at 137 59.2) (size 0.4) (drill 0.2) (layers F.Cu B.Cu) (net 1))
 (via (at 135.8 61) (size 0.4) (drill 0.2) (layers F.Cu B.Cu) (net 1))
 (via (at 135.2 62.8) (size 0.4) (drill 0.2) (layers F.Cu B.Cu) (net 1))
 (via (at 134.6 62.8) (size 0.4) (drill 0.2) (layers F.Cu B.Cu) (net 1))
 (via (at 139.4 58.6) (size 0.4) (drill 0.2) (layers F.Cu B.Cu) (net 1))
 (via (at 140.6 59.8) (size 0.4) (drill 0.2) (layers F.Cu B.Cu) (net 1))
 (via (at 149.6 52.6) (size 0.4) (drill 0.2) (layers F.Cu B.Cu) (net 1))
 (via (at 149.6 51.4) (size 0.4) (drill 0.2) (layers F.Cu B.Cu) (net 1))
 (via (at 149.6 50.8) (size 0.4) (drill 0.2) (layers F.Cu B.Cu) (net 1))
 (via (at 150.8 51.4) (size 0.4) (drill 0.2) (layers F.Cu B.Cu) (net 1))
 (via (at 150.8 52.6) (size 0.4) (drill 0.2) (layers F.Cu B.Cu) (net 1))
 (via (at 150.8 50.8) (size 0.4) (drill 0.2) (layers F.Cu B.Cu) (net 1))
 (via (at 152 51.4) (size 0.4) (drill 0.2) (layers F.Cu B.Cu) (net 1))
 (via (at 152 52.6) (size 0.4) (drill 0.2) (layers F.Cu B.Cu) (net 1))
 (via (at 152 50.8) (size 0.4) (drill 0.2) (layers F.Cu B.Cu) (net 1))
 (via (at 135.8 53.2) (size 0.4) (drill 0.2) (layers F.Cu B.Cu) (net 1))
 (via (at 135.8 54.4) (size 0.4) (drill 0.2) (layers F.Cu B.Cu) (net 1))
 (via (at 137 54.4) (size 0.4) (drill 0.2) (layers F.Cu B.Cu) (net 1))
 (via (at 137 53.2) (size 0.4) (drill 0.2) (layers F.Cu B.Cu) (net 1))
 (via (at 138.2 53.2) (size 0.4) (drill 0.2) (layers F.Cu B.Cu) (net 1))
 (via (at 138.4 62.8) (size 0.4) (drill 0.2) (layers F.Cu B.Cu) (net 1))
 (via (at 138.4 62.2) (size 0.4) (drill 0.2) (layers F.Cu B.Cu) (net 1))
 (via (at 138.4 61) (size 0.4) (drill 0.2) (layers F.Cu B.Cu) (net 1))
 (via (at 147.2 52.6) (size 0.4) (drill 0.2) (layers F.Cu B.Cu) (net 1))
 (via (at 146 52.6) (size 0.4) (drill 0.2) (layers F.Cu B.Cu) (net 1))
 (via (at 141.2 62.8) (size 0.4) (drill 0.2) (layers F.Cu B.Cu) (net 1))
 (via (at 141.8 61.6) (size 0.4) (drill 0.2) (layers F.Cu B.Cu) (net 1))
 (via (at 141.8 62.8) (size 0.4) (drill 0.2) (layers F.Cu B.Cu) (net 1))
 (via (at 141.2 61.6) (size 0.4) (drill 0.2) (layers F.Cu B.Cu) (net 1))
 (segment (start 137 60.75) (end 136 59.75) (width 0.5) (layer F.Cu) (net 5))
 (segment (start 137 60.75) (end 137 62.52499) (width 0.5) (layer F.Cu) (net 5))
 (segment (start 136 59.75) (end 134.57501 59.75) (width 0.5) (layer F.Cu) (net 5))
 (segment (start 139.75 60.5) (end 137 57.75) (width 0.5) (layer F.Cu) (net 4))
 (segment (start 139.75 60.5) (end 139.75 62.52499) (width 0.5) (layer F.Cu) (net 4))
 (segment (start 137 57.75) (end 134.57501 57.75) (width 0.5) (layer F.Cu) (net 4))
 (segment (start 143.25 60.5) (end 138.5 55.75) (width 0.5) (layer F.Cu) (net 3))
 (segment (start 143.25 60.5) (end 143.25 62.52499) (width 0.5) (layer F.Cu) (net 3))
 (segment (start 138.5 55.75) (end 134.57501 55.75) (width 0.5) (layer F.Cu) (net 3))
 (segment (start 151.25 59.25) (end 151.25 57.22) (width 0.5) (layer F.Cu) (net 6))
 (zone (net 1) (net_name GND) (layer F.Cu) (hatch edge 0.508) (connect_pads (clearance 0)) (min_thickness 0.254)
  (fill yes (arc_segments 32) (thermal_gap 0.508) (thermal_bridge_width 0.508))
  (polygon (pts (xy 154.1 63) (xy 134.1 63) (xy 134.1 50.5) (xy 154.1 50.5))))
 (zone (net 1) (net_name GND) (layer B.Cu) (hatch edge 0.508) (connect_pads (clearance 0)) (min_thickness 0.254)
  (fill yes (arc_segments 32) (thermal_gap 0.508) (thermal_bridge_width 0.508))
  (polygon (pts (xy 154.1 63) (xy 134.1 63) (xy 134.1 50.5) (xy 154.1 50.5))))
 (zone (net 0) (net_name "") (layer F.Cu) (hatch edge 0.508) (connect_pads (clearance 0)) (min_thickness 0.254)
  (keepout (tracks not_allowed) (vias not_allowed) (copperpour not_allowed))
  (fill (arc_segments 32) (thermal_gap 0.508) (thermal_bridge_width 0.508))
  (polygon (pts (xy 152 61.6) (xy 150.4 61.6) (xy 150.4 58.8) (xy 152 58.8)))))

